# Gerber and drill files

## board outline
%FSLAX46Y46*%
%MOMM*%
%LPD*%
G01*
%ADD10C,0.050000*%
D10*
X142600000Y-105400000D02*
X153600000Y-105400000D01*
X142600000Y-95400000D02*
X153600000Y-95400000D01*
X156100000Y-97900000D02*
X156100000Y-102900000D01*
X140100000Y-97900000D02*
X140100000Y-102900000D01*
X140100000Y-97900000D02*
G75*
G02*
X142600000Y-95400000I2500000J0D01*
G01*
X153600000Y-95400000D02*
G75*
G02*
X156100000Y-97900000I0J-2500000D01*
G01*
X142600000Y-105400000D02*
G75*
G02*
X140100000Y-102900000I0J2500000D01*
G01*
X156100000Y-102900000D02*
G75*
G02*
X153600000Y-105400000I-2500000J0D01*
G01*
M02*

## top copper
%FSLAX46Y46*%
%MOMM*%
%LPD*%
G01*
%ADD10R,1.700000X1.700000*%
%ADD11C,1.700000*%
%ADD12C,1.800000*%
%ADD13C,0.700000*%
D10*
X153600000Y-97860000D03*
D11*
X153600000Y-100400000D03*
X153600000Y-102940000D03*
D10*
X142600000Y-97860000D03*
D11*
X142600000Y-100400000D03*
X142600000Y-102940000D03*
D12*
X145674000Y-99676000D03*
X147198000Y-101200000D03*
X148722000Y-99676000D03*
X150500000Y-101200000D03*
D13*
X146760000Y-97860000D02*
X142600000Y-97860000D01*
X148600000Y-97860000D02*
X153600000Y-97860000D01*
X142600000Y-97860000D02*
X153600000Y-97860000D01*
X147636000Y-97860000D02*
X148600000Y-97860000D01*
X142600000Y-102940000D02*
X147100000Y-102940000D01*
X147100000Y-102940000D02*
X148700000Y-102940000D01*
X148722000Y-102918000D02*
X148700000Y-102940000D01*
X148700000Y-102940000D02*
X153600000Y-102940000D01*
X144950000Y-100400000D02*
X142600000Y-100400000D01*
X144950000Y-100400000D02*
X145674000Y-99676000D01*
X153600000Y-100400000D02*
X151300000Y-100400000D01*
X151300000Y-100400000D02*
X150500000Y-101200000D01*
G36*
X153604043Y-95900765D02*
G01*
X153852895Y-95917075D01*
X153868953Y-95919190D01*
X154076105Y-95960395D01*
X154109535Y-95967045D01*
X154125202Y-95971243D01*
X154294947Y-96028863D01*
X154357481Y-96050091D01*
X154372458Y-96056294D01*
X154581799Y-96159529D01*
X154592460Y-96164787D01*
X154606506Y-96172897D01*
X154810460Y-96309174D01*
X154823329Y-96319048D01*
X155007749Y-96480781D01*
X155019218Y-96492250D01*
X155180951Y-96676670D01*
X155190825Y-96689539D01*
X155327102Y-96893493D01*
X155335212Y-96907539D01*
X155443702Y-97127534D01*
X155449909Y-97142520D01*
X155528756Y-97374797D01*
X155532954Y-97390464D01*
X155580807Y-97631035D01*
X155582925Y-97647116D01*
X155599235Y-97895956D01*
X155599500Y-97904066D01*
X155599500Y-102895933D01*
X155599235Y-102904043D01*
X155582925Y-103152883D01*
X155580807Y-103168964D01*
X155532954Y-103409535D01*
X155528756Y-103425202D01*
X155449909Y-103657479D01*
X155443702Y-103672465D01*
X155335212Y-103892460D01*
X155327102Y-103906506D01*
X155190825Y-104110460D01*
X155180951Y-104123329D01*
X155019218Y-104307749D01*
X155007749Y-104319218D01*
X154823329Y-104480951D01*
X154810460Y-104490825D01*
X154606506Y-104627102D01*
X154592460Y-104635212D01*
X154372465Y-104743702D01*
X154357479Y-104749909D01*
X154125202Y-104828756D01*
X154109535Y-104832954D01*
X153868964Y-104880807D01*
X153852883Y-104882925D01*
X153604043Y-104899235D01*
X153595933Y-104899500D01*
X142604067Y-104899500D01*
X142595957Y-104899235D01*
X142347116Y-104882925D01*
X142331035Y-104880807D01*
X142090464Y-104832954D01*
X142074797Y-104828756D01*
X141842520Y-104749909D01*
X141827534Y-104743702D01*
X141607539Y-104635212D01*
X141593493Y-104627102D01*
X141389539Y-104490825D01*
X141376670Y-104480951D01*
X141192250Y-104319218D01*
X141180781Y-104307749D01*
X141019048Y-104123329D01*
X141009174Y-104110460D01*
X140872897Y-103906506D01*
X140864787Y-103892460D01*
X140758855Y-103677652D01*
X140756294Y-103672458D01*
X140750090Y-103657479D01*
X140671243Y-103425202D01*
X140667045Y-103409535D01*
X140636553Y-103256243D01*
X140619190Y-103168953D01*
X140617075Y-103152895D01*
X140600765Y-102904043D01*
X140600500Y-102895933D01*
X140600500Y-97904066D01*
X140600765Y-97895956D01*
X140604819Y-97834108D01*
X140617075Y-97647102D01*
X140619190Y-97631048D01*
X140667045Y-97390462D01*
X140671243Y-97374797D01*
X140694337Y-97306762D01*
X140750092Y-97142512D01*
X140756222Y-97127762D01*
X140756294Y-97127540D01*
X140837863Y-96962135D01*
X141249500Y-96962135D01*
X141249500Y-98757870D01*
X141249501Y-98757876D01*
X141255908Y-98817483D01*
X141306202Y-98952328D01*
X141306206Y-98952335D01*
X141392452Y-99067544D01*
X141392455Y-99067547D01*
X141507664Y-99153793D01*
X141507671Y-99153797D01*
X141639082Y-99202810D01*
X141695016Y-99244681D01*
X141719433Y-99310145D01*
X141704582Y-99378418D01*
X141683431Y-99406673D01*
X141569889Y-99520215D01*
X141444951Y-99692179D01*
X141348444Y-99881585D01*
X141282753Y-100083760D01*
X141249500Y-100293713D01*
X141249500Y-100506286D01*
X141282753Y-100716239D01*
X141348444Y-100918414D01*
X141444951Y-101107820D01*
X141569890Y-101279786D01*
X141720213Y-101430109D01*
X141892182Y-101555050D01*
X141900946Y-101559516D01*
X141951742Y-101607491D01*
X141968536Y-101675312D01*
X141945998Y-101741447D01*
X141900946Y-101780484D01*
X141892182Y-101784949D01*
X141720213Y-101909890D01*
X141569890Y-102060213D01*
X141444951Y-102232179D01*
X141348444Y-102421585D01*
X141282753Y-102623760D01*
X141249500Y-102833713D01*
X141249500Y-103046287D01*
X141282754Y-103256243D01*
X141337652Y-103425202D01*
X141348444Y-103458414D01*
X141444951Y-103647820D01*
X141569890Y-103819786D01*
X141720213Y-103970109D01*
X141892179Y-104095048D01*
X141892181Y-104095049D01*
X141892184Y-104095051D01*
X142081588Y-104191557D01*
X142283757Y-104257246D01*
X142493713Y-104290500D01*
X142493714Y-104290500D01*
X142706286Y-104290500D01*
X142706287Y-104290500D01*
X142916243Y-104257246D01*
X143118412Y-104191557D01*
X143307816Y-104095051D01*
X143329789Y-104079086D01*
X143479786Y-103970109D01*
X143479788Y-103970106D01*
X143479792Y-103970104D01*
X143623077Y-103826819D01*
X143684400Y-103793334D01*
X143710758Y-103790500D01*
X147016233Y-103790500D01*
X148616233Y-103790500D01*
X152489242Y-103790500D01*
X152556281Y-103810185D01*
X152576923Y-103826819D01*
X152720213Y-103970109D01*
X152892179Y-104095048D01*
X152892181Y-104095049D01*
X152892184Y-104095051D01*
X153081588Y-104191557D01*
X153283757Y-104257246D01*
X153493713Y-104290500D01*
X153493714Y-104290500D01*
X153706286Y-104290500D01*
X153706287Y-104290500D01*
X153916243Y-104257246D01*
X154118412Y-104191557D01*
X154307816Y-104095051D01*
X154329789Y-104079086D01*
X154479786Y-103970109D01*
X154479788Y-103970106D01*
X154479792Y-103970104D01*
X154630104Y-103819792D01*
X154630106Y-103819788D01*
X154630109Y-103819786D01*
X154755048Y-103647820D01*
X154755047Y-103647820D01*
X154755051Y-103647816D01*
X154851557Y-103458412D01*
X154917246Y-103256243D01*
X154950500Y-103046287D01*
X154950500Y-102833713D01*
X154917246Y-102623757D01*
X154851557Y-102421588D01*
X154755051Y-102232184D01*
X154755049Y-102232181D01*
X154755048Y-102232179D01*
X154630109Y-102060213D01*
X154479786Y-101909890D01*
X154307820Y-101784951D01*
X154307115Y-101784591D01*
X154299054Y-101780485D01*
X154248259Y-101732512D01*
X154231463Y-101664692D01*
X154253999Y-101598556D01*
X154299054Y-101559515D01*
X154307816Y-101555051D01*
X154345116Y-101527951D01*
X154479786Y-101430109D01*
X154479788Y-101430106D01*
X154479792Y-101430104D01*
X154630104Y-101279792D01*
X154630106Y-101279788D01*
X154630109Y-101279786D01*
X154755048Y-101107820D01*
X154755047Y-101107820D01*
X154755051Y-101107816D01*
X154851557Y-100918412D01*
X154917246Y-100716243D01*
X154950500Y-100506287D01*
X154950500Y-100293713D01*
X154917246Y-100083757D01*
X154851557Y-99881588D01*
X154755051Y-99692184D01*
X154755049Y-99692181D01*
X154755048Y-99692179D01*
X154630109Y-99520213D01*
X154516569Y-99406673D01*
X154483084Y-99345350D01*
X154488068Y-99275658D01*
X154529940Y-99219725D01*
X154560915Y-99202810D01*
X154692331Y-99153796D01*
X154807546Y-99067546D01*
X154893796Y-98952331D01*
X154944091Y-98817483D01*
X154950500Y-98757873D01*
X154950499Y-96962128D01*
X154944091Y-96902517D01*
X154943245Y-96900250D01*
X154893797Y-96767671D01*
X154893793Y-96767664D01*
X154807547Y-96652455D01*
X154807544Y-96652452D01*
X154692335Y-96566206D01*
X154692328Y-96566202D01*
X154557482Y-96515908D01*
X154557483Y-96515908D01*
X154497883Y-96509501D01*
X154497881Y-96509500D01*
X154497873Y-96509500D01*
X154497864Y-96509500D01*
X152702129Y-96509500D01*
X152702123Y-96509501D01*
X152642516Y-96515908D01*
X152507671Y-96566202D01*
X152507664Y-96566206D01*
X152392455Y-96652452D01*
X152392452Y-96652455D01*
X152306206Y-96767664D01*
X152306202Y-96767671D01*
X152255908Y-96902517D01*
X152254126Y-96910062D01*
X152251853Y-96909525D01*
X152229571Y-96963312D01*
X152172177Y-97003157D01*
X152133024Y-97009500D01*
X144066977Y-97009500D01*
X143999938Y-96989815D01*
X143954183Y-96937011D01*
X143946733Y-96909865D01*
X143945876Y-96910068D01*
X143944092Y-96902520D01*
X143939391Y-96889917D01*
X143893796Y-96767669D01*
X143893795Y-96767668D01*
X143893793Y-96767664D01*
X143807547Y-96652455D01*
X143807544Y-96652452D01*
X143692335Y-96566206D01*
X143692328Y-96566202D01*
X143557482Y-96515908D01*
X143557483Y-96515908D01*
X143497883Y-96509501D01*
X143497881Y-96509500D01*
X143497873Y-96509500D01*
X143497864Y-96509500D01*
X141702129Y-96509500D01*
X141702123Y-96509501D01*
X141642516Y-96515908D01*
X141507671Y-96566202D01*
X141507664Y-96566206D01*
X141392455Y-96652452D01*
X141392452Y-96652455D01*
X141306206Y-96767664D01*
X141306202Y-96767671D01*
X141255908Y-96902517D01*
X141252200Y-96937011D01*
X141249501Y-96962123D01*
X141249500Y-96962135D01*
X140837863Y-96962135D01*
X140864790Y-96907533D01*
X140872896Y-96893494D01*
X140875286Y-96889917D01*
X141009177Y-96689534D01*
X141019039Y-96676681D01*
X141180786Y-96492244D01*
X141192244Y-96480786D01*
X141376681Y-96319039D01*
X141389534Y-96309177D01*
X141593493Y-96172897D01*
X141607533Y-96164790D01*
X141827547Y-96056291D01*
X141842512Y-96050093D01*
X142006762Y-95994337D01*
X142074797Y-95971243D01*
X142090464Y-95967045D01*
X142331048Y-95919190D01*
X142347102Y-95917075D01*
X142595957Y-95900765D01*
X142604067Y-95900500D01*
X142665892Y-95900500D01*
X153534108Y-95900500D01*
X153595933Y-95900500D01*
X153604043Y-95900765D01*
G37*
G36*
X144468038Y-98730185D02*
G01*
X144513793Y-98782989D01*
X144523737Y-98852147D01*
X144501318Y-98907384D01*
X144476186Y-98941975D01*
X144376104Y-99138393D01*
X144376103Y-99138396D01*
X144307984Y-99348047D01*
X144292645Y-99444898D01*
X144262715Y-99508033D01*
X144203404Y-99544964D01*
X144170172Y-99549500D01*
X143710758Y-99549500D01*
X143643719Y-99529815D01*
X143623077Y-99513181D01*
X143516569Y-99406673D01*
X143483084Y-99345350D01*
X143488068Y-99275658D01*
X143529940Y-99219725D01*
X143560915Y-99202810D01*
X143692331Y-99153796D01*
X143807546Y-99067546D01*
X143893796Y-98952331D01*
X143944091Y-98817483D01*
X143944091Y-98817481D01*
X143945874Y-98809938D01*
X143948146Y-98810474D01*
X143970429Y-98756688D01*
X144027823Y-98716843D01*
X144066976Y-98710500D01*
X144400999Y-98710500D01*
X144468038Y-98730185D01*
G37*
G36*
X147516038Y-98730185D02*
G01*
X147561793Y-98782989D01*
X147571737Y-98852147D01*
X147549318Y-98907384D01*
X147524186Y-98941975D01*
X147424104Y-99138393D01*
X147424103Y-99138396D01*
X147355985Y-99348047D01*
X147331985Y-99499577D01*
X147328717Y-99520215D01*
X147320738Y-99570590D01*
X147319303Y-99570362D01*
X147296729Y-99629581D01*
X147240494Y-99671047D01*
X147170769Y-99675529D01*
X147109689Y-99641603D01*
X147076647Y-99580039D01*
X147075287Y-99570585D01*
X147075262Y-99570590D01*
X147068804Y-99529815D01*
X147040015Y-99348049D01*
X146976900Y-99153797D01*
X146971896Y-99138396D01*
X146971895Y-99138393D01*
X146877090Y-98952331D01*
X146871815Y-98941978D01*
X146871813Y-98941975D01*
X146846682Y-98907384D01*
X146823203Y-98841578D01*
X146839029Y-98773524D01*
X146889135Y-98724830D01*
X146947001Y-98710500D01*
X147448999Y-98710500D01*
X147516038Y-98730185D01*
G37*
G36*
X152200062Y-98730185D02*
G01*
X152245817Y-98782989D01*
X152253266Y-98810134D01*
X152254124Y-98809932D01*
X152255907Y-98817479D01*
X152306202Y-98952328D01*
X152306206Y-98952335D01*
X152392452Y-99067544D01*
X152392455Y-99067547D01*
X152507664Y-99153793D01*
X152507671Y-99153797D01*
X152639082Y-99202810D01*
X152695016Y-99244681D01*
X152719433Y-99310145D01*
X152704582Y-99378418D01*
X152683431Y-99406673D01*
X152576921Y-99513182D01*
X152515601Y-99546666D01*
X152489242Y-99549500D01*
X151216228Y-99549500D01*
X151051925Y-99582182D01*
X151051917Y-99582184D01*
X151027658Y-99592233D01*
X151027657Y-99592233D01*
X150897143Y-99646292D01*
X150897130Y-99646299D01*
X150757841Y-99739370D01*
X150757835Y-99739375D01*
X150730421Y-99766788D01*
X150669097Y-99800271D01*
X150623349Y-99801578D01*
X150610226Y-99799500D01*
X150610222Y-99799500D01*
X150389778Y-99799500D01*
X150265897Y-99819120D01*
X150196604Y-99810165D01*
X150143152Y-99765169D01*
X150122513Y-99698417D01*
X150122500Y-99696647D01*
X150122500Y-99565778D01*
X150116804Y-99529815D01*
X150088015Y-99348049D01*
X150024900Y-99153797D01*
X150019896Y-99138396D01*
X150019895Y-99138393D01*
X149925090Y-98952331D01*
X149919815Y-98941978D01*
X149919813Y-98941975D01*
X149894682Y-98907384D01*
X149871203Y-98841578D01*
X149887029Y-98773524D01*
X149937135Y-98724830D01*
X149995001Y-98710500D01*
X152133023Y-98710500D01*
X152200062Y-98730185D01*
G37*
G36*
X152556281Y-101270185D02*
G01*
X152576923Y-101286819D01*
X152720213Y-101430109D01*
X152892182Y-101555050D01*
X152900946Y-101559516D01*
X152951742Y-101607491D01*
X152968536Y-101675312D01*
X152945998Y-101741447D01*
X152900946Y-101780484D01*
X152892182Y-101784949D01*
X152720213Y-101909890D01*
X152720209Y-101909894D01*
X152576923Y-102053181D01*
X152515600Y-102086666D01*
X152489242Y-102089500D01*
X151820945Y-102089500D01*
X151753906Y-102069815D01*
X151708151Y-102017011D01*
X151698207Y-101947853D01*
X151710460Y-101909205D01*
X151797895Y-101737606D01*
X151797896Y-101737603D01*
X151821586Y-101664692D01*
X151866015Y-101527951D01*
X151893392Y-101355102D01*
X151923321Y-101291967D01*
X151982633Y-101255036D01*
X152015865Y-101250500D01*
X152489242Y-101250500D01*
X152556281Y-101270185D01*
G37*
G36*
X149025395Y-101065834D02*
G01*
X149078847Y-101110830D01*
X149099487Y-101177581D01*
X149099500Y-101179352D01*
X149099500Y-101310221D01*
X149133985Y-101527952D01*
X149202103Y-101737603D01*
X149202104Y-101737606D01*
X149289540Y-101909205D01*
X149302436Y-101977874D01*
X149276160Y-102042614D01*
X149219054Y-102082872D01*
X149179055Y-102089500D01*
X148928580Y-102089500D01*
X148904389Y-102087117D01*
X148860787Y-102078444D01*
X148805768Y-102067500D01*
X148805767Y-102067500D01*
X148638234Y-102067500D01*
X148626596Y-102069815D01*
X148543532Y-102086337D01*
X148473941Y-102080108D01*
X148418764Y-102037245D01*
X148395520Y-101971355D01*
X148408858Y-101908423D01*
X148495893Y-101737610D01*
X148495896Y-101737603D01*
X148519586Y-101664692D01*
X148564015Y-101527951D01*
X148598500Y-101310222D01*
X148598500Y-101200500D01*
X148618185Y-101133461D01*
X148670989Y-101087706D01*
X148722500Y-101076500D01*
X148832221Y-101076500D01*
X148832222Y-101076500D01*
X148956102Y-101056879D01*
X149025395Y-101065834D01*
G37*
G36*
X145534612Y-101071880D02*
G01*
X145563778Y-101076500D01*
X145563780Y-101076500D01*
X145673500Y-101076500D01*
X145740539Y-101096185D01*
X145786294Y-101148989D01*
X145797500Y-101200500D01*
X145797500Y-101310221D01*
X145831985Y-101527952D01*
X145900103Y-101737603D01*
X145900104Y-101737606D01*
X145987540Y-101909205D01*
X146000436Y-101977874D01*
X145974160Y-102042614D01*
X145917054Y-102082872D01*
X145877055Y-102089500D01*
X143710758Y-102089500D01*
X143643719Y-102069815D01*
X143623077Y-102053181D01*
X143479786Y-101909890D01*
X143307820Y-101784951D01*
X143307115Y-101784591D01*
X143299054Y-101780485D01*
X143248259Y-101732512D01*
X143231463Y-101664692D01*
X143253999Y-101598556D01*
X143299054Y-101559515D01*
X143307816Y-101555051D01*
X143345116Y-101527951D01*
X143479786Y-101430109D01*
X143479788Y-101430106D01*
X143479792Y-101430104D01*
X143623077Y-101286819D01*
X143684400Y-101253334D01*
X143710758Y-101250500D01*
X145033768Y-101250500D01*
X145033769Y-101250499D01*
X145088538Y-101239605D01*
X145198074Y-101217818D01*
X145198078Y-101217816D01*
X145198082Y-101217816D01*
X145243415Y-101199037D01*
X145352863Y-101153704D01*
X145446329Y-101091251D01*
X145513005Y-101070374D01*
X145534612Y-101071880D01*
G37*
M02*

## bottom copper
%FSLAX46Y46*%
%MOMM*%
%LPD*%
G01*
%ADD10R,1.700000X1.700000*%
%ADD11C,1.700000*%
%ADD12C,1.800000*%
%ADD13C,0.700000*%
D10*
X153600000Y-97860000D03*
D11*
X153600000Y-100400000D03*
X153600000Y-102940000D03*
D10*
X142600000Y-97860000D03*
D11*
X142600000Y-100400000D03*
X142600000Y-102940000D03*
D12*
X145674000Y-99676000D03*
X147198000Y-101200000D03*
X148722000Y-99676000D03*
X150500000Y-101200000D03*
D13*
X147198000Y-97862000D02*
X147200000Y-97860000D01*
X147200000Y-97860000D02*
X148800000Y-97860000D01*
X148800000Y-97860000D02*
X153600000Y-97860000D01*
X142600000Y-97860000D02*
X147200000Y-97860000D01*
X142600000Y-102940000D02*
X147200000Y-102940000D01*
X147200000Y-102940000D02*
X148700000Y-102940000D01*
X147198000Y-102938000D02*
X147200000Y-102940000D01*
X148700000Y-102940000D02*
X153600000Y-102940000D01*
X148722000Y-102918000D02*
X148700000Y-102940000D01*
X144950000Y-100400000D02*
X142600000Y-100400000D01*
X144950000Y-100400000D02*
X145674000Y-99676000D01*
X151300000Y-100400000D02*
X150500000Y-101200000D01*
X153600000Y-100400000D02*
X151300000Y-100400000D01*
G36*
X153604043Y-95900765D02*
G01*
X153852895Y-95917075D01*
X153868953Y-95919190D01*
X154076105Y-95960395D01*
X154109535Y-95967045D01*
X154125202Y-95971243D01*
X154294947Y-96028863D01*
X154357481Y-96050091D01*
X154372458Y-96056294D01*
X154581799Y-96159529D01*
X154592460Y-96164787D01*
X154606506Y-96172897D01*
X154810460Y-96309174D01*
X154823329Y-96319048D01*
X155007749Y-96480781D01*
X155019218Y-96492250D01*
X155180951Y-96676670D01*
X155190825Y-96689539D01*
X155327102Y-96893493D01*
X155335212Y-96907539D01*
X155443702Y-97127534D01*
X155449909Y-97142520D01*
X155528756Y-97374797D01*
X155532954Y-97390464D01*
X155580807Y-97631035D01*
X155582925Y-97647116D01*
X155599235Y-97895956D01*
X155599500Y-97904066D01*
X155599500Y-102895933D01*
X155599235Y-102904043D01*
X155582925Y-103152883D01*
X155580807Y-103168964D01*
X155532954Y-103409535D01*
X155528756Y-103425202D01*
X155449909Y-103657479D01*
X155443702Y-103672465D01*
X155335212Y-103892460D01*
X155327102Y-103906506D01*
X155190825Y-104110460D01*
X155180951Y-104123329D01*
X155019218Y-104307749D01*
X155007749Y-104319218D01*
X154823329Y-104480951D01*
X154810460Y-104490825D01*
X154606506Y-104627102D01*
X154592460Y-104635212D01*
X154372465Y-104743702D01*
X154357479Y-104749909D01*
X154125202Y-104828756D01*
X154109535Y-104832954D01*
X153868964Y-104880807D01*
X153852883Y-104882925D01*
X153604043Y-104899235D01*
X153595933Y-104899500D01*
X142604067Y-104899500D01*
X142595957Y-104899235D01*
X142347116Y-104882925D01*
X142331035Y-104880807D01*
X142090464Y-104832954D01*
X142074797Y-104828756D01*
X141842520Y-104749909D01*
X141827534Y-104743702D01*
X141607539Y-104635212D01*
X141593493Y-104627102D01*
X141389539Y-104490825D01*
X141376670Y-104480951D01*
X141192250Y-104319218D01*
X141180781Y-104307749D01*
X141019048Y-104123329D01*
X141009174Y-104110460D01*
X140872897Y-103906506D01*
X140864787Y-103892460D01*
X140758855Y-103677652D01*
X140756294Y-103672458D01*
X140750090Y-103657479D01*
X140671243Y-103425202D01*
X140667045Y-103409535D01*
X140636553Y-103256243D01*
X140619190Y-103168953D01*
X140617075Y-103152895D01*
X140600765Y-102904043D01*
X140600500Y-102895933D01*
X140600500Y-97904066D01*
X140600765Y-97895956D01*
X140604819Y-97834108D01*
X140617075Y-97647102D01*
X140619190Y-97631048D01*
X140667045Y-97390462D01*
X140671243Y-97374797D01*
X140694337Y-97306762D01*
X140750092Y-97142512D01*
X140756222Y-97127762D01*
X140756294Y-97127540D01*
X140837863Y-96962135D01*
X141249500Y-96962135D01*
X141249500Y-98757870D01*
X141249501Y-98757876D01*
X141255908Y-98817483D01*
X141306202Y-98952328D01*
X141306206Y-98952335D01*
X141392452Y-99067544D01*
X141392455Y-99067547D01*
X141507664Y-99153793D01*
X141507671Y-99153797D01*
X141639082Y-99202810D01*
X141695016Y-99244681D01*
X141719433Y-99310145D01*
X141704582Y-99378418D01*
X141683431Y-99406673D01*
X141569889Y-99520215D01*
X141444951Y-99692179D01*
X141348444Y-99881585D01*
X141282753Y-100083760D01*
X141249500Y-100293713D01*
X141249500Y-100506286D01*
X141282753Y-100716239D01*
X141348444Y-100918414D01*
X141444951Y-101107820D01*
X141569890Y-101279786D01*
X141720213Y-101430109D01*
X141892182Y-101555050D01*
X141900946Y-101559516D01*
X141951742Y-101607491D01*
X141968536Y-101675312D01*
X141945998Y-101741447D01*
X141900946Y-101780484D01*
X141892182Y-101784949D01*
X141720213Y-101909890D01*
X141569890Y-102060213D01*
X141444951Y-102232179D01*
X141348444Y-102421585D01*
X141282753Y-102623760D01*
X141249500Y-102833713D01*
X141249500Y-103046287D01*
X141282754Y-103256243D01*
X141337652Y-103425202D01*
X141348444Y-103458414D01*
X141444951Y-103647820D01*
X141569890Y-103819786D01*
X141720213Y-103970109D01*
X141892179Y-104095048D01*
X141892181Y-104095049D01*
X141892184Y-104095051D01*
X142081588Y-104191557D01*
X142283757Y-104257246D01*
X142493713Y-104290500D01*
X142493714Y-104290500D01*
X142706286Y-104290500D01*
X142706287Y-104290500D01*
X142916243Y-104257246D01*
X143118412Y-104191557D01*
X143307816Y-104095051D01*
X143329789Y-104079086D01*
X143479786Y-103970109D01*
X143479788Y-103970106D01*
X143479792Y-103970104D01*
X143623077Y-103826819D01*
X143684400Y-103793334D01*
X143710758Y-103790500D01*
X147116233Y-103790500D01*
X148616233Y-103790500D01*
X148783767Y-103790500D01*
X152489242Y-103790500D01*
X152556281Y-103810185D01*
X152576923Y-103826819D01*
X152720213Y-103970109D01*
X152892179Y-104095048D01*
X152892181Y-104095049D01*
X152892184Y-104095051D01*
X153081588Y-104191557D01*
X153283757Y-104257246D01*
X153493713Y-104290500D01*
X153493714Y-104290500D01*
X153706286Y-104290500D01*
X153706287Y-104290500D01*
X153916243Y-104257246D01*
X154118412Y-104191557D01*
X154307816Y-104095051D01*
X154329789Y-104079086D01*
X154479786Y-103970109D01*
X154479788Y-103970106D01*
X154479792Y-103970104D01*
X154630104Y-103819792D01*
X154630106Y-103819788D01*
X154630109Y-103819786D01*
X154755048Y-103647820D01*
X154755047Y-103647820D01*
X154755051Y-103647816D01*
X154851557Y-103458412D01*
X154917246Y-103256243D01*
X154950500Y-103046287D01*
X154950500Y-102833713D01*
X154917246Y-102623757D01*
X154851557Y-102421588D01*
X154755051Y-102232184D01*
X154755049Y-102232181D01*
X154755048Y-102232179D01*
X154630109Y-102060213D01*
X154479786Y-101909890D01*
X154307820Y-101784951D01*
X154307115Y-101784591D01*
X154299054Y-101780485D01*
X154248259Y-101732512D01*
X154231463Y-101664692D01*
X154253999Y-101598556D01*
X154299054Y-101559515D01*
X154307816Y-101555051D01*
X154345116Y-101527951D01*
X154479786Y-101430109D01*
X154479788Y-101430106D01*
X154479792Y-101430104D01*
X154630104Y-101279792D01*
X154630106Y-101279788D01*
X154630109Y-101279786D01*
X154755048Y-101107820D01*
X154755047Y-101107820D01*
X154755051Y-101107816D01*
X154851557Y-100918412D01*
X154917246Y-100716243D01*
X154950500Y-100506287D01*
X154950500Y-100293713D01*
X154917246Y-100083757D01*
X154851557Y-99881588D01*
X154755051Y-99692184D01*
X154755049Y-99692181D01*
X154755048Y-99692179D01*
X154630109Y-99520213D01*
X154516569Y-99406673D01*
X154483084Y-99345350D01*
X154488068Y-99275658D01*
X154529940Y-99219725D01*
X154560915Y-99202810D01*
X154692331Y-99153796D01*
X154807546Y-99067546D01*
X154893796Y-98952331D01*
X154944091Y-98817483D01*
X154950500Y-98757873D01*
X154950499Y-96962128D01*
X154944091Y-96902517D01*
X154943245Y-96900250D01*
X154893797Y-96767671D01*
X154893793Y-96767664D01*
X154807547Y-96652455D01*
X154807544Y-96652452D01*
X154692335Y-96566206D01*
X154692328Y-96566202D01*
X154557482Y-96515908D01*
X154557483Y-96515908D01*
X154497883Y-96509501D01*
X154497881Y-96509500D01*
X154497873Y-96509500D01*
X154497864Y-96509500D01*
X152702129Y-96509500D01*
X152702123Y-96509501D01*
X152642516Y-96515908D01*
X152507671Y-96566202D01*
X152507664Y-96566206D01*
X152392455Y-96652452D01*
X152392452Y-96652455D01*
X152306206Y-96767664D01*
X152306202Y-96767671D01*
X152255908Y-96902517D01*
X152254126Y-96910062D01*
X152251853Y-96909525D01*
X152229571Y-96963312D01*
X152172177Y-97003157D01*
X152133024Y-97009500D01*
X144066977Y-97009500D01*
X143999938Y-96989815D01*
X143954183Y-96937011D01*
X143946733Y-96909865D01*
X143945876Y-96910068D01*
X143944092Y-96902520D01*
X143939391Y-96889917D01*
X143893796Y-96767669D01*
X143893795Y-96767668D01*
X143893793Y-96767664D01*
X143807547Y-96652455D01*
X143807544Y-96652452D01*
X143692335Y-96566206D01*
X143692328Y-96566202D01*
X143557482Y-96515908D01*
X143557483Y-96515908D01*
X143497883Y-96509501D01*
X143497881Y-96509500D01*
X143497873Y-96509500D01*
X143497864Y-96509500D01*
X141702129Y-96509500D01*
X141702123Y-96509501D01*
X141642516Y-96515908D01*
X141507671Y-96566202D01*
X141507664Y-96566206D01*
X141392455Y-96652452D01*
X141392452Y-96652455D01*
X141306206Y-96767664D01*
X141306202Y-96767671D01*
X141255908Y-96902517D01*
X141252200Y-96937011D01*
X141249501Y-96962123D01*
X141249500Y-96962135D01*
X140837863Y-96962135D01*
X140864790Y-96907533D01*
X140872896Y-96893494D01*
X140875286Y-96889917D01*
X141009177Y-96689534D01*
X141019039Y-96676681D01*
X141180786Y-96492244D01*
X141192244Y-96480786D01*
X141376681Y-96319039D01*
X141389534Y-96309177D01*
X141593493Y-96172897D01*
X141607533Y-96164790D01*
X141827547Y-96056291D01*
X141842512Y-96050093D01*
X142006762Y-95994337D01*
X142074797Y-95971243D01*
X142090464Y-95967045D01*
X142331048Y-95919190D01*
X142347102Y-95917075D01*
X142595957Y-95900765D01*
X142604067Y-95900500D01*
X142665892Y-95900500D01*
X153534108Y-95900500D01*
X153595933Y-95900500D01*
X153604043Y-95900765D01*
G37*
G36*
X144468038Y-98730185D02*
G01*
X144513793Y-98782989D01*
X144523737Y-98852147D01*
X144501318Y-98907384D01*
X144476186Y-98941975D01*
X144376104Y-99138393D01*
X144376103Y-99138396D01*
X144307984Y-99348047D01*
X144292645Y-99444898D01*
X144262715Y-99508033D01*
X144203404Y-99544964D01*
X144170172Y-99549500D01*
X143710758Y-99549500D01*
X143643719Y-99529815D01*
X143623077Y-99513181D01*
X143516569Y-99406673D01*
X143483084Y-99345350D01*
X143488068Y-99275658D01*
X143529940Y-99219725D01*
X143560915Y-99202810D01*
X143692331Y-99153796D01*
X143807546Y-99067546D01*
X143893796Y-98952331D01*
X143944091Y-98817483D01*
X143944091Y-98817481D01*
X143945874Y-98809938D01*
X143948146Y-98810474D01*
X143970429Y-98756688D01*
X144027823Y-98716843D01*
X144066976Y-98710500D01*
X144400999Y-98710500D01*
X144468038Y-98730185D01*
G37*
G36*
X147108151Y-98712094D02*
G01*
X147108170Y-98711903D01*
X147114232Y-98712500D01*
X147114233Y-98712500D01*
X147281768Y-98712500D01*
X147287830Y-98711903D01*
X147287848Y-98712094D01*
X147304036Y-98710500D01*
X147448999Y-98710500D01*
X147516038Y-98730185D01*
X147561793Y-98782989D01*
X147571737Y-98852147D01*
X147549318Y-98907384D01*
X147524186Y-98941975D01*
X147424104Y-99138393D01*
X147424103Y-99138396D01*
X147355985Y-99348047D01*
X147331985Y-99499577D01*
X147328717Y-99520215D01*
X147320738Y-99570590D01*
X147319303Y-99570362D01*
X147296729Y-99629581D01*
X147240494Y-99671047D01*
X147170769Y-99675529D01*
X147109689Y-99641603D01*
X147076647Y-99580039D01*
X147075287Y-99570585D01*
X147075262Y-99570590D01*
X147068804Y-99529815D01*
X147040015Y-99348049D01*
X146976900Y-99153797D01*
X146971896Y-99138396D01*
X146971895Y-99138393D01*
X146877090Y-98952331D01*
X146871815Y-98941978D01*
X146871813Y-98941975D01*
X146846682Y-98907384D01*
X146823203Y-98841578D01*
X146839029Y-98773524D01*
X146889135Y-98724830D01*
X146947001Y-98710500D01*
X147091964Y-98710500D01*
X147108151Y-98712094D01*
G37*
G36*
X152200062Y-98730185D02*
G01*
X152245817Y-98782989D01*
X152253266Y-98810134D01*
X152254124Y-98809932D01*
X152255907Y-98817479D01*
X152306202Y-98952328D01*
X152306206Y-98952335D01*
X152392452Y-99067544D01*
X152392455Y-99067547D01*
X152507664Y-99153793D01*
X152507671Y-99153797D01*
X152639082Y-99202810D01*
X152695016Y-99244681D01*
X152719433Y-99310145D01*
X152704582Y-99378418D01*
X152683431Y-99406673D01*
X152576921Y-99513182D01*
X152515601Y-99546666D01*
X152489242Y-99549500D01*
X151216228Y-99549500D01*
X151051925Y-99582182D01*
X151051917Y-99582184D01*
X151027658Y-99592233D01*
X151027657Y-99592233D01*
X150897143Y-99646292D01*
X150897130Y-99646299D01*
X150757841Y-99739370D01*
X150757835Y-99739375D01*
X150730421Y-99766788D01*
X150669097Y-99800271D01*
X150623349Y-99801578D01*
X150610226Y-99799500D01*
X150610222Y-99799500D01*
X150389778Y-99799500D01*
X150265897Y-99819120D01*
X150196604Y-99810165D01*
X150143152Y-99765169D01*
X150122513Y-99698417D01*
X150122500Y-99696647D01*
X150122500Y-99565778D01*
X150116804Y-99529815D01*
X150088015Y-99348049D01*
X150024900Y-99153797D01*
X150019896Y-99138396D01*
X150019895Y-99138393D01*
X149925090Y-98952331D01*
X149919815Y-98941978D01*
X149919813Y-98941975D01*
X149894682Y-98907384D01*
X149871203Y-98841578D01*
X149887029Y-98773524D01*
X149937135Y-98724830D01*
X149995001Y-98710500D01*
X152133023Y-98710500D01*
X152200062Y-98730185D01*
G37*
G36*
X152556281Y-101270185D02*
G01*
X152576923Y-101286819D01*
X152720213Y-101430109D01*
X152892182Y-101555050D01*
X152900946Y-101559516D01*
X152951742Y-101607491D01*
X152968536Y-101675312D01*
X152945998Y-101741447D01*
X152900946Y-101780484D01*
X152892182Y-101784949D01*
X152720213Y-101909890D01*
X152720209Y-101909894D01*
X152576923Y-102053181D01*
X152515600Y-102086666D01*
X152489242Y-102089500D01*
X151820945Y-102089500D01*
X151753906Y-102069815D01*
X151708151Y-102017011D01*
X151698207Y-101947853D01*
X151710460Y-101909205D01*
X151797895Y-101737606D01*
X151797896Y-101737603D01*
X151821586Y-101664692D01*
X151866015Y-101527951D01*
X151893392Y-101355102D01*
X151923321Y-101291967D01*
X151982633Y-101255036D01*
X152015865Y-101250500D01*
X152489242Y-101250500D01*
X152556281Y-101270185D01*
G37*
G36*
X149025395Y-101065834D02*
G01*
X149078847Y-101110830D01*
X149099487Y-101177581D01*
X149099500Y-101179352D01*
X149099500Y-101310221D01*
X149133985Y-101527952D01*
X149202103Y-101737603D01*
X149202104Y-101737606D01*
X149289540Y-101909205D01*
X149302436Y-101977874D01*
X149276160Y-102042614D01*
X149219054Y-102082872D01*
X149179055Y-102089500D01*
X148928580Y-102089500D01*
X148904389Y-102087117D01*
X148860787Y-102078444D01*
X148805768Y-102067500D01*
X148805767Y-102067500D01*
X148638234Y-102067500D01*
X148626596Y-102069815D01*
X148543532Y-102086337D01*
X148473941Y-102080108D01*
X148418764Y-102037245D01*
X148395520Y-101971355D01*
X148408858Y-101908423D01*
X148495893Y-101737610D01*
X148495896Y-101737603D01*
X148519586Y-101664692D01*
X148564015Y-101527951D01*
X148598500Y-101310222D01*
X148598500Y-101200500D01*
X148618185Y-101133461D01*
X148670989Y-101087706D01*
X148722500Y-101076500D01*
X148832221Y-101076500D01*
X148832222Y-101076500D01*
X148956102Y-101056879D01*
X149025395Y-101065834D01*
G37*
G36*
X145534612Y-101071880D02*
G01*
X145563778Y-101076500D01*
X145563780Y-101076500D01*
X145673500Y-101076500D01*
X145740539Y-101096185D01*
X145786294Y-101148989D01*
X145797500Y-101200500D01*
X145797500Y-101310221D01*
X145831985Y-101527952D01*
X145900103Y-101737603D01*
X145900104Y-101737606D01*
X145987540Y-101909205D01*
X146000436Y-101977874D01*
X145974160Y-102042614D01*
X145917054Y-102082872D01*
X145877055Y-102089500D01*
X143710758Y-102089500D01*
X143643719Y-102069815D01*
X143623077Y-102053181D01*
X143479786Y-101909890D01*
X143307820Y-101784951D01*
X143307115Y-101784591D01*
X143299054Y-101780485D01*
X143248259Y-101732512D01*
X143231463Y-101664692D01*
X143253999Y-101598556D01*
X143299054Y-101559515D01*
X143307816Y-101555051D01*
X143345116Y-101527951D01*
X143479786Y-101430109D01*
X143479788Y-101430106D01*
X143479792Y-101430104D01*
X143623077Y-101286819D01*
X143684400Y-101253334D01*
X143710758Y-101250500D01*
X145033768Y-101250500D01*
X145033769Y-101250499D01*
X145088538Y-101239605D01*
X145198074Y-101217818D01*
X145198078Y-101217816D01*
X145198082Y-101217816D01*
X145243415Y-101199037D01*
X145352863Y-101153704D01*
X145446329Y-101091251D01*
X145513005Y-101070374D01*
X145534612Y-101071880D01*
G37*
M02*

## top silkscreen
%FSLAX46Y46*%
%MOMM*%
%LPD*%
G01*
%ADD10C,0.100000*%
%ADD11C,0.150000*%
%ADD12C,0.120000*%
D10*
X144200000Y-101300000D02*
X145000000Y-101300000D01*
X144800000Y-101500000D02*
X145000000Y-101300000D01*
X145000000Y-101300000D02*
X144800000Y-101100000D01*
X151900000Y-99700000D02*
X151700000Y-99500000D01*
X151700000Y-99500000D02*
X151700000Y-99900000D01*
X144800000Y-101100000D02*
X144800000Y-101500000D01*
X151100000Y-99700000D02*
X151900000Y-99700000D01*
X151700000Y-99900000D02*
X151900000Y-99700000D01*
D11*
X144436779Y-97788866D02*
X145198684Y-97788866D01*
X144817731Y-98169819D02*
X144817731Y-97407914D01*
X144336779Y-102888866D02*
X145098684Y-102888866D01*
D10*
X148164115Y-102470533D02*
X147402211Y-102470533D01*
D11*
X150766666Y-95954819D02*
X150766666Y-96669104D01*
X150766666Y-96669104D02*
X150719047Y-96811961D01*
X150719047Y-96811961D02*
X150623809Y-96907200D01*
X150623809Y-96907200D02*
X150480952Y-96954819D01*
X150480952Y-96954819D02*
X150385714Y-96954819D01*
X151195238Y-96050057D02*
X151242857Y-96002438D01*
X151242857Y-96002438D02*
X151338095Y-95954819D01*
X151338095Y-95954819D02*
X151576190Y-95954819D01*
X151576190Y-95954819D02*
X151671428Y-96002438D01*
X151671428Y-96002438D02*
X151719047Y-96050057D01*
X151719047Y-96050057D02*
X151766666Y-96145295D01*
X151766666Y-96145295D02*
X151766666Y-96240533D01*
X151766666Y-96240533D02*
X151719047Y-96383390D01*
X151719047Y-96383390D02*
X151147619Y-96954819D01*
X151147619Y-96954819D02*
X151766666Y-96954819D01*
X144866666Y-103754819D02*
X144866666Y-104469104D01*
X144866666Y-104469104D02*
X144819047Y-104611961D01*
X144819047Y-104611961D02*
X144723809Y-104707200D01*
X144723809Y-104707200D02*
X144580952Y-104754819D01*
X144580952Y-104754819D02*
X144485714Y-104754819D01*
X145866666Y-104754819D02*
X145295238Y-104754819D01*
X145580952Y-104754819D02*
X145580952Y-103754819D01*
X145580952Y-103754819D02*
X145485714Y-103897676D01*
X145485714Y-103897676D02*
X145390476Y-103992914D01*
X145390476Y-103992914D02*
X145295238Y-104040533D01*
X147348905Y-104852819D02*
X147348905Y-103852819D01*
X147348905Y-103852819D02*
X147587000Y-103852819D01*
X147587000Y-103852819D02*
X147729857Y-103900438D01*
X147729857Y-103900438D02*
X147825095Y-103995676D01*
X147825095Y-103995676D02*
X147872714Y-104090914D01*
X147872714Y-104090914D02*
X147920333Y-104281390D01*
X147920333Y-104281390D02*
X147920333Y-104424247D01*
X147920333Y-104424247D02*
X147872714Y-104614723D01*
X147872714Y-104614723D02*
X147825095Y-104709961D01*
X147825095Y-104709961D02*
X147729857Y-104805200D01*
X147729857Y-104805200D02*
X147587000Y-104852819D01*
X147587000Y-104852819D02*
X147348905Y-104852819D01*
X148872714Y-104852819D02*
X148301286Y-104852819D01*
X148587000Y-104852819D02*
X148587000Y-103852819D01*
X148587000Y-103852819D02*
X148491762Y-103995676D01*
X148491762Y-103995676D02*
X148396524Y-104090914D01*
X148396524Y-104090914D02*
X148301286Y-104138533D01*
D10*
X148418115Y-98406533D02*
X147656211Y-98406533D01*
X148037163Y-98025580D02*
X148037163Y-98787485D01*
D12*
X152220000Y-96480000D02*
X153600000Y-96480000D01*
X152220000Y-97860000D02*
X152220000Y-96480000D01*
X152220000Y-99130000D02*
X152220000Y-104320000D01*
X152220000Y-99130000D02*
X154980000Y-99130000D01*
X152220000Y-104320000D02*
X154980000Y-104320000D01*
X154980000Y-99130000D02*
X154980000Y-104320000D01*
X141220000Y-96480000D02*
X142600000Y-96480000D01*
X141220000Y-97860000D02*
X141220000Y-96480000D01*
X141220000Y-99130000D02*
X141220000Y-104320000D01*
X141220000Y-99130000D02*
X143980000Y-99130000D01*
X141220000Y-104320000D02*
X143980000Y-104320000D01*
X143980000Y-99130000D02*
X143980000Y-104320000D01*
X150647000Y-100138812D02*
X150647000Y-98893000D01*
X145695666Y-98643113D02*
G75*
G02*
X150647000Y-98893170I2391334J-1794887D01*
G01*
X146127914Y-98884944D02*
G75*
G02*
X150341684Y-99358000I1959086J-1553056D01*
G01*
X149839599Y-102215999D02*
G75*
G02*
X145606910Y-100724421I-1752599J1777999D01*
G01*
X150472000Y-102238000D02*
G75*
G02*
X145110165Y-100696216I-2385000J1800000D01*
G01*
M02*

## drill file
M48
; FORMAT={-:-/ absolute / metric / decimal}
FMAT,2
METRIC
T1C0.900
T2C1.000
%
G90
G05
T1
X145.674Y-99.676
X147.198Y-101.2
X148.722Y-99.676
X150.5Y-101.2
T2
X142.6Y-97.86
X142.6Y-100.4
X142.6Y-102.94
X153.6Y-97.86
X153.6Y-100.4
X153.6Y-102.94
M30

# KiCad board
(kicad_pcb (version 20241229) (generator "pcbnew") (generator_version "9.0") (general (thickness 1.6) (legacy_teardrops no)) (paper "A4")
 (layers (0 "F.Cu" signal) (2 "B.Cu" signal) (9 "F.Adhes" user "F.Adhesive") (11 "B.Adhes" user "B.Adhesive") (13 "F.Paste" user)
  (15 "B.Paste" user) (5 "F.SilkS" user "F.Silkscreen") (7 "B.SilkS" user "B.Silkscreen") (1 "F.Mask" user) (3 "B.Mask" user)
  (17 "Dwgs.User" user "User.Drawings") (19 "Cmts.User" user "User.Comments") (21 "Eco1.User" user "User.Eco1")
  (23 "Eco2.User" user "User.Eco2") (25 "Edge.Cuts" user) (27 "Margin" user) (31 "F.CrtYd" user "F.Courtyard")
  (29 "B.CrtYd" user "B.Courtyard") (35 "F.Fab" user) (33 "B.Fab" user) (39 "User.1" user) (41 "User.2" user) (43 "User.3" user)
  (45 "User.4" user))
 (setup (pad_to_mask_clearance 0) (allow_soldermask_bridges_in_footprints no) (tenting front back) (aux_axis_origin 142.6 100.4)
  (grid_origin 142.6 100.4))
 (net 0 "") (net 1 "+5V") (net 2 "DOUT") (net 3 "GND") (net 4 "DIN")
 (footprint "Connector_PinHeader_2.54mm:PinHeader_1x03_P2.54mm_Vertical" (layer "F.Cu") (at 153.6 97.86)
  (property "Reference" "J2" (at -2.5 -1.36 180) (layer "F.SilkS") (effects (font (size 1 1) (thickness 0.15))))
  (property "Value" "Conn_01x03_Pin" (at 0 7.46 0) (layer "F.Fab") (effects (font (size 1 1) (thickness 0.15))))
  (fp_line (start -1.38 -1.38) (end 0 -1.38) (stroke (width 0.12) (type solid)) (layer "F.SilkS"))
  (fp_line (start -1.38 0) (end -1.38 -1.38) (stroke (width 0.12) (type solid)) (layer "F.SilkS"))
  (fp_line (start -1.38 1.27) (end -1.38 6.46) (stroke (width 0.12) (type solid)) (layer "F.SilkS"))
  (fp_line (start -1.38 1.27) (end 1.38 1.27) (stroke (width 0.12) (type solid)) (layer "F.SilkS"))
  (fp_line (start -1.38 6.46) (end 1.38 6.46) (stroke (width 0.12) (type solid)) (layer "F.SilkS"))
  (fp_line (start 1.38 1.27) (end 1.38 6.46) (stroke (width 0.12) (type solid)) (layer "F.SilkS"))
  (pad "1" thru_hole rect (at 0 0) (size 1.7 1.7) (drill 1) (layers "*.Cu" "*.Mask") (remove_unused_layers no) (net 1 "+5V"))
  (pad "2" thru_hole circle (at 0 2.54) (size 1.7 1.7) (drill 1) (layers "*.Cu" "*.Mask") (remove_unused_layers no) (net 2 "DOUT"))
  (pad "3" thru_hole circle (at 0 5.08) (size 1.7 1.7) (drill 1) (layers "*.Cu" "*.Mask") (remove_unused_layers no) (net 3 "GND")))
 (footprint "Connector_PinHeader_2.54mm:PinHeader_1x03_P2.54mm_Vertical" (layer "F.Cu") (at 142.6 97.86)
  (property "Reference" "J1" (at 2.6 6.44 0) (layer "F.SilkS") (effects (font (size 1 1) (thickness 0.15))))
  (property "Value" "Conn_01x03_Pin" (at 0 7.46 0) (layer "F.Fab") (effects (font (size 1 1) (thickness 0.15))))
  (fp_line (start -1.38 -1.38) (end 0 -1.38) (stroke (width 0.12) (type solid)) (layer "F.SilkS"))
  (fp_line (start -1.38 0) (end -1.38 -1.38) (stroke (width 0.12) (type solid)) (layer "F.SilkS"))
  (fp_line (start -1.38 1.27) (end -1.38 6.46) (stroke (width 0.12) (type solid)) (layer "F.SilkS"))
  (fp_line (start -1.38 1.27) (end 1.38 1.27) (stroke (width 0.12) (type solid)) (layer "F.SilkS"))
  (fp_line (start -1.38 6.46) (end 1.38 6.46) (stroke (width 0.12) (type solid)) (layer "F.SilkS"))
  (fp_line (start 1.38 1.27) (end 1.38 6.46) (stroke (width 0.12) (type solid)) (layer "F.SilkS"))
  (pad "1" thru_hole rect (at 0 0) (size 1.7 1.7) (drill 1) (layers "*.Cu" "*.Mask") (remove_unused_layers no) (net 1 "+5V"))
  (pad "2" thru_hole circle (at 0 2.54) (size 1.7 1.7) (drill 1) (layers "*.Cu" "*.Mask") (remove_unused_layers no) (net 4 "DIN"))
  (pad "3" thru_hole circle (at 0 5.08) (size 1.7 1.7) (drill 1) (layers "*.Cu" "*.Mask") (remove_unused_layers no) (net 3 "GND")))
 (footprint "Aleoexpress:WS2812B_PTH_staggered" (layer "F.Cu") (at 150.5 101.2 180)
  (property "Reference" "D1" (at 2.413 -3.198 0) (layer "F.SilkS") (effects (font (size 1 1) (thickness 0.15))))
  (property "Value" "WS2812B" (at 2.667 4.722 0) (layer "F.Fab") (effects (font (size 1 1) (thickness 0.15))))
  (fp_line (start -0.147 1.061188) (end -0.147 2.307) (stroke (width 0.12) (type solid)) (layer "F.SilkS"))
  (fp_arc (start 4.804334 2.556887) (mid 2.262188 3.748194) (end -0.147 2.30683) (stroke (width 0.12) (type solid)) (layer "F.SilkS"))
  (fp_arc (start 4.372086 2.315056) (mid 2.134091 3.246393) (end 0.158316 1.842) (stroke (width 0.12) (type solid)) (layer "F.SilkS"))
  (fp_arc (start 0.660401 -1.015999) (mid 3.242766 -1.592649) (end 4.89309 0.475579) (stroke (width 0.12) (type solid)) (layer "F.SilkS"))
  (fp_arc (start 0.028 -1.038) (mid 3.238737 -2.109652) (end 5.389836 0.503784) (stroke (width 0.12) (type solid)) (layer "F.SilkS"))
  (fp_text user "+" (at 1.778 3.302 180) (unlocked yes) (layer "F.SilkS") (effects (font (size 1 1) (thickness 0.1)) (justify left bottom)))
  (pad "1" thru_hole circle (at 4.826 1.524 180) (size 1.8 1.8) (drill 0.9) (layers "*.Cu" "*.Mask") (remove_unused_layers no) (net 4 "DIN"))
  (pad "2" thru_hole circle (at 3.302 0 180) (size 1.8 1.8) (drill 0.9) (layers "*.Cu" "*.Mask") (remove_unused_layers no) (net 3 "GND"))
  (pad "3" thru_hole circle (at 1.778 1.524 180) (size 1.8 1.8) (drill 0.9) (layers "*.Cu" "*.Mask") (remove_unused_layers no) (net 1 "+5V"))
  (pad "4" thru_hole circle (at 0 0 180) (size 1.8 1.8) (drill 0.9) (layers "*.Cu" "*.Mask") (remove_unused_layers no) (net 2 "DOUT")))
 (gr_line (start 144.2 101.3) (end 145 101.3) (stroke (width 0.1) (type default)) (layer "F.SilkS"))
 (gr_line (start 144.8 101.5) (end 145 101.3) (stroke (width 0.1) (type default)) (layer "F.SilkS"))
 (gr_line (start 145 101.3) (end 144.8 101.1) (stroke (width 0.1) (type default)) (layer "F.SilkS"))
 (gr_line (start 151.9 99.7) (end 151.7 99.5) (stroke (width 0.1) (type default)) (layer "F.SilkS"))
 (gr_line (start 151.7 99.5) (end 151.7 99.9) (stroke (width 0.1) (type default)) (layer "F.SilkS"))
 (gr_line (start 144.8 101.1) (end 144.8 101.5) (stroke (width 0.1) (type default)) (layer "F.SilkS"))
 (gr_line (start 151.1 99.7) (end 151.9 99.7) (stroke (width 0.1) (type default)) (layer "F.SilkS"))
 (gr_line (start 151.7 99.9) (end 151.9 99.7) (stroke (width 0.1) (type default)) (layer "F.SilkS"))
 (gr_line (start 142.6 105.4) (end 153.6 105.4) (stroke (width 0.05) (type default)) (layer "Edge.Cuts"))
 (gr_line (start 142.6 95.4) (end 153.6 95.4) (stroke (width 0.05) (type default)) (layer "Edge.Cuts"))
 (gr_line (start 156.1 97.9) (end 156.1 102.9) (stroke (width 0.05) (type default)) (layer "Edge.Cuts"))
 (gr_line (start 140.1 97.9) (end 140.1 102.9) (stroke (width 0.05) (type default)) (layer "Edge.Cuts"))
 (gr_arc (start 140.1 97.9) (mid 140.832233 96.132233) (end 142.6 95.4) (stroke (width 0.05) (type default)) (layer "Edge.Cuts"))
 (gr_arc (start 153.6 95.4) (mid 155.367767 96.132233) (end 156.1 97.9) (stroke (width 0.05) (type default)) (layer "Edge.Cuts"))
 (gr_arc (start 142.6 105.4) (mid 140.832233 104.667767) (end 140.1 102.9) (stroke (width 0.05) (type default)) (layer "Edge.Cuts"))
 (gr_arc (start 156.1 102.9) (mid 155.367767 104.667767) (end 153.6 105.4) (stroke (width 0.05) (type default)) (layer "Edge.Cuts"))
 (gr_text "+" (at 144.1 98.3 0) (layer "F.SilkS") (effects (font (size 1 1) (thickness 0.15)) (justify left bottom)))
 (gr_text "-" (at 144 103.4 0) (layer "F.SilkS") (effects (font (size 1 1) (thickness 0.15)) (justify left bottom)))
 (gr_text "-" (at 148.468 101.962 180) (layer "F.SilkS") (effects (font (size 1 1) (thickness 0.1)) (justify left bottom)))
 (segment (start 146.76 97.86) (end 142.6 97.86) (width 0.7) (layer "F.Cu") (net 1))
 (segment (start 148.6 97.86) (end 153.6 97.86) (width 0.7) (layer "F.Cu") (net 1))
 (segment (start 142.6 97.86) (end 153.6 97.86) (width 0.7) (layer "F.Cu") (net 1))
 (segment (start 147.636 97.86) (end 148.6 97.86) (width 0.7) (layer "F.Cu") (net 1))
 (segment (start 147.198 97.862) (end 147.2 97.86) (width 0.7) (layer "B.Cu") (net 1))
 (segment (start 147.2 97.86) (end 148.8 97.86) (width 0.7) (layer "B.Cu") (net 1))
 (segment (start 148.8 97.86) (end 153.6 97.86) (width 0.7) (layer "B.Cu") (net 1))
 (segment (start 142.6 97.86) (end 147.2 97.86) (width 0.7) (layer "B.Cu") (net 1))
 (segment (start 142.6 102.94) (end 147.1 102.94) (width 0.7) (layer "F.Cu") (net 3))
 (segment (start 147.1 102.94) (end 148.7 102.94) (width 0.7) (layer "F.Cu") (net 3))
 (segment (start 148.722 102.918) (end 148.7 102.94) (width 0.7) (layer "F.Cu") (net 3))
 (segment (start 148.7 102.94) (end 153.6 102.94) (width 0.7) (layer "F.Cu") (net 3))
 (segment (start 142.6 102.94) (end 147.2 102.94) (width 0.7) (layer "B.Cu") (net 3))
 (segment (start 147.2 102.94) (end 148.7 102.94) (width 0.7) (layer "B.Cu") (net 3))
 (segment (start 147.198 102.938) (end 147.2 102.94) (width 0.7) (layer "B.Cu") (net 3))
 (segment (start 148.7 102.94) (end 153.6 102.94) (width 0.7) (layer "B.Cu") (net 3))
 (segment (start 148.722 102.918) (end 148.7 102.94) (width 0.7) (layer "B.Cu") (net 3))
 (segment (start 144.95 100.4) (end 142.6 100.4) (width 0.7) (layer "F.Cu") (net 4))
 (segment (start 144.95 100.4) (end 145.674 99.676) (width 0.7) (layer "F.Cu") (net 4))
 (segment (start 144.95 100.4) (end 142.6 100.4) (width 0.7) (layer "B.Cu") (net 4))
 (segment (start 144.95 100.4) (end 145.674 99.676) (width 0.7) (layer "B.Cu") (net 4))
 (segment (start 153.6 100.4) (end 151.3 100.4) (width 0.7) (layer "F.Cu") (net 2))
 (segment (start 151.3 100.4) (end 150.5 101.2) (width 0.7) (layer "F.Cu") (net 2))
 (segment (start 151.3 100.4) (end 150.5 101.2) (width 0.7) (layer "B.Cu") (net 2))
 (segment (start 153.6 100.4) (end 151.3 100.4) (width 0.7) (layer "B.Cu") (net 2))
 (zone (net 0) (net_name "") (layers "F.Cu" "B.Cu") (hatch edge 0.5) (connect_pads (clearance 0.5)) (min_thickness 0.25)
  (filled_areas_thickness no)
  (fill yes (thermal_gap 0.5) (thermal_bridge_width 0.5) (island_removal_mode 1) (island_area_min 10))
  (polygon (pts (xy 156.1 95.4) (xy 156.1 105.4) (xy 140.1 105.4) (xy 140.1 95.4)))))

